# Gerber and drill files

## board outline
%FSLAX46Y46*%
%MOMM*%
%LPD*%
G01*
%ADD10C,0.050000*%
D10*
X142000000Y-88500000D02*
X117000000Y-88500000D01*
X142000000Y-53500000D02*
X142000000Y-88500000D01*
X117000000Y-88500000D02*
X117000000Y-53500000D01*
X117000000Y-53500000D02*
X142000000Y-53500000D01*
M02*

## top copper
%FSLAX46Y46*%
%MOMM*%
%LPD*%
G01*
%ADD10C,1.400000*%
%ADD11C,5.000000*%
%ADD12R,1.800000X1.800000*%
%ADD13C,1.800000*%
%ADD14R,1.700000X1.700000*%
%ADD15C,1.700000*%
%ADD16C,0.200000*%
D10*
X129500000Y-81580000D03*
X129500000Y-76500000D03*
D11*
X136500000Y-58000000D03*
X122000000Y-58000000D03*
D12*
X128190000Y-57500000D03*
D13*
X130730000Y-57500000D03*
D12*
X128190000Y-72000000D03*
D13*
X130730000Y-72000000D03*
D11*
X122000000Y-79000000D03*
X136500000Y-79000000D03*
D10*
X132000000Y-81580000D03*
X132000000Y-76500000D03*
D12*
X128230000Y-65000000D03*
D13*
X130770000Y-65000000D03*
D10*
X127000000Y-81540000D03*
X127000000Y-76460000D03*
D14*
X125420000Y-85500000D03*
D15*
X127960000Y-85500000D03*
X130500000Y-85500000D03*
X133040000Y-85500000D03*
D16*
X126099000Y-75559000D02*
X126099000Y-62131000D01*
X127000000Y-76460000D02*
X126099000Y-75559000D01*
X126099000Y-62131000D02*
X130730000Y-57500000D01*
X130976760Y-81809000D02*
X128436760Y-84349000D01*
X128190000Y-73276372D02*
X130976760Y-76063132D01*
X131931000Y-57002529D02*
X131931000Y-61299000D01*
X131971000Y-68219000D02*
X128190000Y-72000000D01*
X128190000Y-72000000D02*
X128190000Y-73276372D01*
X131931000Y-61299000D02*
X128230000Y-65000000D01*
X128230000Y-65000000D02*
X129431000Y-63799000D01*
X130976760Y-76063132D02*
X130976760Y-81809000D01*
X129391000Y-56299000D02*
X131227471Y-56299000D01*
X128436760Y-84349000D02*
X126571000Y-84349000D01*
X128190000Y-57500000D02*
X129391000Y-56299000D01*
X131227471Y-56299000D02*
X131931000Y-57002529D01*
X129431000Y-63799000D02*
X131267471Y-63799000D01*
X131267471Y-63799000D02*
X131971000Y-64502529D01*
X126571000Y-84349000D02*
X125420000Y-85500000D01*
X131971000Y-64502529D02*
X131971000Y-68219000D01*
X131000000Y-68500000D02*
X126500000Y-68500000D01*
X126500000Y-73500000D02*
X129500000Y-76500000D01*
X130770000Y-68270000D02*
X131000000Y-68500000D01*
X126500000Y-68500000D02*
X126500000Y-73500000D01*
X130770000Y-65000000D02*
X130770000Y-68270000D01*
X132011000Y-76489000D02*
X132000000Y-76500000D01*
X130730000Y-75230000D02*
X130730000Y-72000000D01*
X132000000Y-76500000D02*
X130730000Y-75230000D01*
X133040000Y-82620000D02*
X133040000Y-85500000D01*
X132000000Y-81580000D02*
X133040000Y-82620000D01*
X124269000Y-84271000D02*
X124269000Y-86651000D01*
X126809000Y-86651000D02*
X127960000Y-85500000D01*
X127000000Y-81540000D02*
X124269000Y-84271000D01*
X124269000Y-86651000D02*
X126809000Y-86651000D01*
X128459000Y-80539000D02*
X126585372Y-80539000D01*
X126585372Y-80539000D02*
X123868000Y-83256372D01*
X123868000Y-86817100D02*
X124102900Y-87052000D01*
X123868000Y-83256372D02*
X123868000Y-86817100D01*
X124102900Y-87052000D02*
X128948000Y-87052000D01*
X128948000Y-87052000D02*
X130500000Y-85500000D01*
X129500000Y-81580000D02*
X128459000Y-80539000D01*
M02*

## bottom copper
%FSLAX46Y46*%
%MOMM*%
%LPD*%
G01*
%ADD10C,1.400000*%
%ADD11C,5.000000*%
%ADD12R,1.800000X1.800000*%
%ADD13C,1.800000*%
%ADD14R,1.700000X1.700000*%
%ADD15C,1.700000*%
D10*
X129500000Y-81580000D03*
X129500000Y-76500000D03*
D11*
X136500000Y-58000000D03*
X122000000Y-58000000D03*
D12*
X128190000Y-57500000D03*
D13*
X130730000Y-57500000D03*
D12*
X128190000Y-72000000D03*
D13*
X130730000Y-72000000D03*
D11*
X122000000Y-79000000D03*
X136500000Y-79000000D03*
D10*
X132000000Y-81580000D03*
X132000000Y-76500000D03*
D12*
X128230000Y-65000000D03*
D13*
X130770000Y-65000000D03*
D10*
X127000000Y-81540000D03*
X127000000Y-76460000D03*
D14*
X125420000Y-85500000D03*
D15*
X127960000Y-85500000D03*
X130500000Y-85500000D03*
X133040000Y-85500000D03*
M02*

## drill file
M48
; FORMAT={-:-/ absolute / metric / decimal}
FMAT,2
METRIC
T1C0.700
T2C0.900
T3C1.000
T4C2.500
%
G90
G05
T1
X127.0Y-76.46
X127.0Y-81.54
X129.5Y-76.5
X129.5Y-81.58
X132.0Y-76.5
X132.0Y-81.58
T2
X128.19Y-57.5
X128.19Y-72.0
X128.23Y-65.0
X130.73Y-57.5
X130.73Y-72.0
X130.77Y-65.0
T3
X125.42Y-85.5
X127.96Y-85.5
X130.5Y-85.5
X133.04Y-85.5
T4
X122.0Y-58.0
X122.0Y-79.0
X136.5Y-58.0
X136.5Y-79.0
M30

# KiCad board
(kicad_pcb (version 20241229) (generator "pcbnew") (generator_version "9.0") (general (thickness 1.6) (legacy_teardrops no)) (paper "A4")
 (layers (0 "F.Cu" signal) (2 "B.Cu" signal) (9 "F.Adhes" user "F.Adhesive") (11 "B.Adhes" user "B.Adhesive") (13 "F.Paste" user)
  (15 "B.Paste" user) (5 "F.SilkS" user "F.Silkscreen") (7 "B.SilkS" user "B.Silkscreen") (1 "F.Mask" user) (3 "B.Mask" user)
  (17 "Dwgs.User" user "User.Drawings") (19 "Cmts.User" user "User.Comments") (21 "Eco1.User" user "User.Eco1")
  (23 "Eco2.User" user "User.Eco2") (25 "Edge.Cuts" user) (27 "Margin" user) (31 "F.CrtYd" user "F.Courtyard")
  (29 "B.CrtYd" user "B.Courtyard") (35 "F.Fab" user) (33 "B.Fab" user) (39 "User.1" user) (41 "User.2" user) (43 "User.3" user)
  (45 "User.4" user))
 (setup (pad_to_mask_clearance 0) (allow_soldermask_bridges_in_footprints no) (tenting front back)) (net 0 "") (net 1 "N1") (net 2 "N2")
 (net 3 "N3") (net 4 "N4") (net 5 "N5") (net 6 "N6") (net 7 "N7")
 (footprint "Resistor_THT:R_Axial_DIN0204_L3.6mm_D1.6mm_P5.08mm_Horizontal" (layer "F.Cu") (at 129.5 81.58 90)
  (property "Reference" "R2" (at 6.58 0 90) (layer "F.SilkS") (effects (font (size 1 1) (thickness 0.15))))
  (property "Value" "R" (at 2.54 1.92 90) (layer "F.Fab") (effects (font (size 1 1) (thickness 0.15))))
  (pad "1" thru_hole circle (at 0 0 90) (size 1.4 1.4) (drill 0.7) (layers "*.Cu" "*.Mask") (remove_unused_layers no) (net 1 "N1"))
  (pad "2" thru_hole circle (at 5.08 0 90) (size 1.4 1.4) (drill 0.7) (layers "*.Cu" "*.Mask") (remove_unused_layers no) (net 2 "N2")))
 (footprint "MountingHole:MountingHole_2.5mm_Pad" (layer "F.Cu") (at 136.5 58)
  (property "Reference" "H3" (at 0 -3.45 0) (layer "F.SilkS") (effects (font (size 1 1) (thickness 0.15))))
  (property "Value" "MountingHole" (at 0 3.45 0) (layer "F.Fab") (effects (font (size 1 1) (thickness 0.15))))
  (pad "1" thru_hole circle (at 0 0) (size 5 5) (drill 2.5) (layers "*.Cu" "*.Mask") (remove_unused_layers no) (zone_connect 2)))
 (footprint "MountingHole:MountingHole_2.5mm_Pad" (layer "F.Cu") (at 122 58)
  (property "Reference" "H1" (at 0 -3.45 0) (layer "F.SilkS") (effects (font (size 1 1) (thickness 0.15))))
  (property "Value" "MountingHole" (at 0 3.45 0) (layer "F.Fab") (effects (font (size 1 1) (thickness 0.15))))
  (pad "1" thru_hole circle (at 0 0) (size 5 5) (drill 2.5) (layers "*.Cu" "*.Mask") (remove_unused_layers no) (zone_connect 2)))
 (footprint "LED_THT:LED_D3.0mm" (layer "F.Cu") (at 128.19 57.5)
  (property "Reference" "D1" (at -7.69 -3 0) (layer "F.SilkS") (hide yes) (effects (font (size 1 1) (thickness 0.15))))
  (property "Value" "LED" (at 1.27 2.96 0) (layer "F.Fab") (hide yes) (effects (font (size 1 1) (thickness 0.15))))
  (pad "1" thru_hole rect (at 0 0) (size 1.8 1.8) (drill 0.9) (layers "*.Cu" "*.Mask") (remove_unused_layers no) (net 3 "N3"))
  (pad "2" thru_hole circle (at 2.54 0) (size 1.8 1.8) (drill 0.9) (layers "*.Cu" "*.Mask") (remove_unused_layers no) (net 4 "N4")))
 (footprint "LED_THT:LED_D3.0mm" (layer "F.Cu") (at 128.19 72)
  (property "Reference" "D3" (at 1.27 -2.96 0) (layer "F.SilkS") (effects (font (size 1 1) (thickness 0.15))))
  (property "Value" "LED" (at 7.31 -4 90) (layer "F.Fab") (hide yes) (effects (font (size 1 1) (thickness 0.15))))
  (pad "1" thru_hole rect (at 0 0) (size 1.8 1.8) (drill 0.9) (layers "*.Cu" "*.Mask") (remove_unused_layers no) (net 3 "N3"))
  (pad "2" thru_hole circle (at 2.54 0) (size 1.8 1.8) (drill 0.9) (layers "*.Cu" "*.Mask") (remove_unused_layers no) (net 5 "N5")))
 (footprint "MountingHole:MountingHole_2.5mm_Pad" (layer "F.Cu") (at 122 79)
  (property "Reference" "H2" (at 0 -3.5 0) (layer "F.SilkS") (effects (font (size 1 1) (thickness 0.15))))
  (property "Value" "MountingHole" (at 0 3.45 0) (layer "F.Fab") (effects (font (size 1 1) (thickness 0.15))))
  (pad "1" thru_hole circle (at 0 0) (size 5 5) (drill 2.5) (layers "*.Cu" "*.Mask") (remove_unused_layers no) (zone_connect 2)))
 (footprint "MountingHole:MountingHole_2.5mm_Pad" (layer "F.Cu") (at 136.5 79)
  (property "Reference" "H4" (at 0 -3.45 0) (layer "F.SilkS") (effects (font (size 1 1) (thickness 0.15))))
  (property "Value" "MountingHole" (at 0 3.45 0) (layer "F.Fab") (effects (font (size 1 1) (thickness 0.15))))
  (pad "1" thru_hole circle (at 0 0) (size 5 5) (drill 2.5) (layers "*.Cu" "*.Mask") (remove_unused_layers no) (zone_connect 2)))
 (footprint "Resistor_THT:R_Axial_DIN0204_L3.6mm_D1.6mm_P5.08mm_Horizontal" (layer "F.Cu") (at 132 81.58 90)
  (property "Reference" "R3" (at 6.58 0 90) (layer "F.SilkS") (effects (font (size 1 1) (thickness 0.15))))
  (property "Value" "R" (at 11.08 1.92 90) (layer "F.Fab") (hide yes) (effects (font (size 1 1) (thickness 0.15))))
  (pad "1" thru_hole circle (at 0 0 90) (size 1.4 1.4) (drill 0.7) (layers "*.Cu" "*.Mask") (remove_unused_layers no) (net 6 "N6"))
  (pad "2" thru_hole circle (at 5.08 0 90) (size 1.4 1.4) (drill 0.7) (layers "*.Cu" "*.Mask") (remove_unused_layers no) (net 5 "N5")))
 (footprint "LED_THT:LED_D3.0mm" (layer "F.Cu") (at 128.23 65)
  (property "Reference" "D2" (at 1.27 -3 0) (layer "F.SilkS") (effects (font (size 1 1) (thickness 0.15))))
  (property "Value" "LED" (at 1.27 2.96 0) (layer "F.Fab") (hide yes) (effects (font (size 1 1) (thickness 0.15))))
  (pad "1" thru_hole rect (at 0 0) (size 1.8 1.8) (drill 0.9) (layers "*.Cu" "*.Mask") (remove_unused_layers no) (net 3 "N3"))
  (pad "2" thru_hole circle (at 2.54 0) (size 1.8 1.8) (drill 0.9) (layers "*.Cu" "*.Mask") (remove_unused_layers no) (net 2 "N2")))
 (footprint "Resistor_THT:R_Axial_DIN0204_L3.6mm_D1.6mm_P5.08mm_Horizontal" (layer "F.Cu") (at 127 81.54 90)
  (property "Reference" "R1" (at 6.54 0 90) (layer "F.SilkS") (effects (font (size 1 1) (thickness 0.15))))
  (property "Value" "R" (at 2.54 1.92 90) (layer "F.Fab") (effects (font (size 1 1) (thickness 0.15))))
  (pad "1" thru_hole circle (at 0 0 90) (size 1.4 1.4) (drill 0.7) (layers "*.Cu" "*.Mask") (remove_unused_layers no) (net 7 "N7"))
  (pad "2" thru_hole circle (at 5.08 0 90) (size 1.4 1.4) (drill 0.7) (layers "*.Cu" "*.Mask") (remove_unused_layers no) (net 4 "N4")))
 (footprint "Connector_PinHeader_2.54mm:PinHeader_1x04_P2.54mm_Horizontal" (layer "B.Cu") (at 125.42 85.5 -90)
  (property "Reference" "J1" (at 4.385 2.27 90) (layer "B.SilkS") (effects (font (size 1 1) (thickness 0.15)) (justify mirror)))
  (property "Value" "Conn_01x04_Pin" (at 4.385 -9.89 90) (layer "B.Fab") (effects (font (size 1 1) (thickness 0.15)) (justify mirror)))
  (pad "1" thru_hole rect (at 0 0 270) (size 1.7 1.7) (drill 1) (layers "*.Cu" "*.Mask") (remove_unused_layers no) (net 3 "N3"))
  (pad "2" thru_hole circle (at 0 -2.54 270) (size 1.7 1.7) (drill 1) (layers "*.Cu" "*.Mask") (remove_unused_layers no) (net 7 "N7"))
  (pad "3" thru_hole circle (at 0 -5.08 270) (size 1.7 1.7) (drill 1) (layers "*.Cu" "*.Mask") (remove_unused_layers no) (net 1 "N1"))
  (pad "4" thru_hole circle (at 0 -7.62 270) (size 1.7 1.7) (drill 1) (layers "*.Cu" "*.Mask") (remove_unused_layers no) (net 6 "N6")))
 (gr_line (start 142 88.5) (end 117 88.5) (stroke (width 0.05) (type default)) (layer "Edge.Cuts"))
 (gr_line (start 142 53.5) (end 142 88.5) (stroke (width 0.05) (type default)) (layer "Edge.Cuts"))
 (gr_line (start 117 88.5) (end 117 53.5) (stroke (width 0.05) (type default)) (layer "Edge.Cuts"))
 (gr_line (start 117 53.5) (end 142 53.5) (stroke (width 0.05) (type default)) (layer "Edge.Cuts"))
 (segment (start 126.099 75.559) (end 126.099 62.131) (width 0.2) (layer "F.Cu") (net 4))
 (segment (start 127 76.46) (end 126.099 75.559) (width 0.2) (layer "F.Cu") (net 4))
 (segment (start 126.099 62.131) (end 130.73 57.5) (width 0.2) (layer "F.Cu") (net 4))
 (segment (start 130.97676 81.809) (end 128.43676 84.349) (width 0.2) (layer "F.Cu") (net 3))
 (segment (start 128.19 73.276372) (end 130.97676 76.063132) (width 0.2) (layer "F.Cu") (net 3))
 (segment (start 131.931 57.002529) (end 131.931 61.299) (width 0.2) (layer "F.Cu") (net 3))
 (segment (start 131.971 68.219) (end 128.19 72) (width 0.2) (layer "F.Cu") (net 3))
 (segment (start 128.19 72) (end 128.19 73.276372) (width 0.2) (layer "F.Cu") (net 3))
 (segment (start 131.931 61.299) (end 128.23 65) (width 0.2) (layer "F.Cu") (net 3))
 (segment (start 128.23 65) (end 129.431 63.799) (width 0.2) (layer "F.Cu") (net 3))
 (segment (start 130.97676 76.063132) (end 130.97676 81.809) (width 0.2) (layer "F.Cu") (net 3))
 (segment (start 129.391 56.299) (end 131.227471 56.299) (width 0.2) (layer "F.Cu") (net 3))
 (segment (start 128.43676 84.349) (end 126.571 84.349) (width 0.2) (layer "F.Cu") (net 3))
 (segment (start 128.19 57.5) (end 129.391 56.299) (width 0.2) (layer "F.Cu") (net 3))
 (segment (start 131.227471 56.299) (end 131.931 57.002529) (width 0.2) (layer "F.Cu") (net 3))
 (segment (start 129.431 63.799) (end 131.267471 63.799) (width 0.2) (layer "F.Cu") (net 3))
 (segment (start 131.267471 63.799) (end 131.971 64.502529) (width 0.2) (layer "F.Cu") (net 3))
 (segment (start 126.571 84.349) (end 125.42 85.5) (width 0.2) (layer "F.Cu") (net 3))
 (segment (start 131.971 64.502529) (end 131.971 68.219) (width 0.2) (layer "F.Cu") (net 3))
 (segment (start 131 68.5) (end 126.5 68.5) (width 0.2) (layer "F.Cu") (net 2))
 (segment (start 126.5 73.5) (end 129.5 76.5) (width 0.2) (layer "F.Cu") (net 2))
 (segment (start 130.77 68.27) (end 131 68.5) (width 0.2) (layer "F.Cu") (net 2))
 (segment (start 126.5 68.5) (end 126.5 73.5) (width 0.2) (layer "F.Cu") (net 2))
 (segment (start 130.77 65) (end 130.77 68.27) (width 0.2) (layer "F.Cu") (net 2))
 (segment (start 132.011 76.489) (end 132 76.5) (width 0.2) (layer "F.Cu") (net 5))
 (segment (start 130.73 75.23) (end 130.73 72) (width 0.2) (layer "F.Cu") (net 5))
 (segment (start 132 76.5) (end 130.73 75.23) (width 0.2) (layer "F.Cu") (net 5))
 (segment (start 133.04 82.62) (end 133.04 85.5) (width 0.2) (layer "F.Cu") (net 6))
 (segment (start 132 81.58) (end 133.04 82.62) (width 0.2) (layer "F.Cu") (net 6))
 (segment (start 124.269 84.271) (end 124.269 86.651) (width 0.2) (layer "F.Cu") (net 7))
 (segment (start 126.809 86.651) (end 127.96 85.5) (width 0.2) (layer "F.Cu") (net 7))
 (segment (start 127 81.54) (end 124.269 84.271) (width 0.2) (layer "F.Cu") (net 7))
 (segment (start 124.269 86.651) (end 126.809 86.651) (width 0.2) (layer "F.Cu") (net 7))
 (segment (start 128.459 80.539) (end 126.585372 80.539) (width 0.2) (layer "F.Cu") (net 1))
 (segment (start 126.585372 80.539) (end 123.868 83.256372) (width 0.2) (layer "F.Cu") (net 1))
 (segment (start 123.868 86.8171) (end 124.1029 87.052) (width 0.2) (layer "F.Cu") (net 1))
 (segment (start 123.868 83.256372) (end 123.868 86.8171) (width 0.2) (layer "F.Cu") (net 1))
 (segment (start 124.1029 87.052) (end 128.948 87.052) (width 0.2) (layer "F.Cu") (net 1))
 (segment (start 128.948 87.052) (end 130.5 85.5) (width 0.2) (layer "F.Cu") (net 1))
 (segment (start 129.5 81.58) (end 128.459 80.539) (width 0.2) (layer "F.Cu") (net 1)))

